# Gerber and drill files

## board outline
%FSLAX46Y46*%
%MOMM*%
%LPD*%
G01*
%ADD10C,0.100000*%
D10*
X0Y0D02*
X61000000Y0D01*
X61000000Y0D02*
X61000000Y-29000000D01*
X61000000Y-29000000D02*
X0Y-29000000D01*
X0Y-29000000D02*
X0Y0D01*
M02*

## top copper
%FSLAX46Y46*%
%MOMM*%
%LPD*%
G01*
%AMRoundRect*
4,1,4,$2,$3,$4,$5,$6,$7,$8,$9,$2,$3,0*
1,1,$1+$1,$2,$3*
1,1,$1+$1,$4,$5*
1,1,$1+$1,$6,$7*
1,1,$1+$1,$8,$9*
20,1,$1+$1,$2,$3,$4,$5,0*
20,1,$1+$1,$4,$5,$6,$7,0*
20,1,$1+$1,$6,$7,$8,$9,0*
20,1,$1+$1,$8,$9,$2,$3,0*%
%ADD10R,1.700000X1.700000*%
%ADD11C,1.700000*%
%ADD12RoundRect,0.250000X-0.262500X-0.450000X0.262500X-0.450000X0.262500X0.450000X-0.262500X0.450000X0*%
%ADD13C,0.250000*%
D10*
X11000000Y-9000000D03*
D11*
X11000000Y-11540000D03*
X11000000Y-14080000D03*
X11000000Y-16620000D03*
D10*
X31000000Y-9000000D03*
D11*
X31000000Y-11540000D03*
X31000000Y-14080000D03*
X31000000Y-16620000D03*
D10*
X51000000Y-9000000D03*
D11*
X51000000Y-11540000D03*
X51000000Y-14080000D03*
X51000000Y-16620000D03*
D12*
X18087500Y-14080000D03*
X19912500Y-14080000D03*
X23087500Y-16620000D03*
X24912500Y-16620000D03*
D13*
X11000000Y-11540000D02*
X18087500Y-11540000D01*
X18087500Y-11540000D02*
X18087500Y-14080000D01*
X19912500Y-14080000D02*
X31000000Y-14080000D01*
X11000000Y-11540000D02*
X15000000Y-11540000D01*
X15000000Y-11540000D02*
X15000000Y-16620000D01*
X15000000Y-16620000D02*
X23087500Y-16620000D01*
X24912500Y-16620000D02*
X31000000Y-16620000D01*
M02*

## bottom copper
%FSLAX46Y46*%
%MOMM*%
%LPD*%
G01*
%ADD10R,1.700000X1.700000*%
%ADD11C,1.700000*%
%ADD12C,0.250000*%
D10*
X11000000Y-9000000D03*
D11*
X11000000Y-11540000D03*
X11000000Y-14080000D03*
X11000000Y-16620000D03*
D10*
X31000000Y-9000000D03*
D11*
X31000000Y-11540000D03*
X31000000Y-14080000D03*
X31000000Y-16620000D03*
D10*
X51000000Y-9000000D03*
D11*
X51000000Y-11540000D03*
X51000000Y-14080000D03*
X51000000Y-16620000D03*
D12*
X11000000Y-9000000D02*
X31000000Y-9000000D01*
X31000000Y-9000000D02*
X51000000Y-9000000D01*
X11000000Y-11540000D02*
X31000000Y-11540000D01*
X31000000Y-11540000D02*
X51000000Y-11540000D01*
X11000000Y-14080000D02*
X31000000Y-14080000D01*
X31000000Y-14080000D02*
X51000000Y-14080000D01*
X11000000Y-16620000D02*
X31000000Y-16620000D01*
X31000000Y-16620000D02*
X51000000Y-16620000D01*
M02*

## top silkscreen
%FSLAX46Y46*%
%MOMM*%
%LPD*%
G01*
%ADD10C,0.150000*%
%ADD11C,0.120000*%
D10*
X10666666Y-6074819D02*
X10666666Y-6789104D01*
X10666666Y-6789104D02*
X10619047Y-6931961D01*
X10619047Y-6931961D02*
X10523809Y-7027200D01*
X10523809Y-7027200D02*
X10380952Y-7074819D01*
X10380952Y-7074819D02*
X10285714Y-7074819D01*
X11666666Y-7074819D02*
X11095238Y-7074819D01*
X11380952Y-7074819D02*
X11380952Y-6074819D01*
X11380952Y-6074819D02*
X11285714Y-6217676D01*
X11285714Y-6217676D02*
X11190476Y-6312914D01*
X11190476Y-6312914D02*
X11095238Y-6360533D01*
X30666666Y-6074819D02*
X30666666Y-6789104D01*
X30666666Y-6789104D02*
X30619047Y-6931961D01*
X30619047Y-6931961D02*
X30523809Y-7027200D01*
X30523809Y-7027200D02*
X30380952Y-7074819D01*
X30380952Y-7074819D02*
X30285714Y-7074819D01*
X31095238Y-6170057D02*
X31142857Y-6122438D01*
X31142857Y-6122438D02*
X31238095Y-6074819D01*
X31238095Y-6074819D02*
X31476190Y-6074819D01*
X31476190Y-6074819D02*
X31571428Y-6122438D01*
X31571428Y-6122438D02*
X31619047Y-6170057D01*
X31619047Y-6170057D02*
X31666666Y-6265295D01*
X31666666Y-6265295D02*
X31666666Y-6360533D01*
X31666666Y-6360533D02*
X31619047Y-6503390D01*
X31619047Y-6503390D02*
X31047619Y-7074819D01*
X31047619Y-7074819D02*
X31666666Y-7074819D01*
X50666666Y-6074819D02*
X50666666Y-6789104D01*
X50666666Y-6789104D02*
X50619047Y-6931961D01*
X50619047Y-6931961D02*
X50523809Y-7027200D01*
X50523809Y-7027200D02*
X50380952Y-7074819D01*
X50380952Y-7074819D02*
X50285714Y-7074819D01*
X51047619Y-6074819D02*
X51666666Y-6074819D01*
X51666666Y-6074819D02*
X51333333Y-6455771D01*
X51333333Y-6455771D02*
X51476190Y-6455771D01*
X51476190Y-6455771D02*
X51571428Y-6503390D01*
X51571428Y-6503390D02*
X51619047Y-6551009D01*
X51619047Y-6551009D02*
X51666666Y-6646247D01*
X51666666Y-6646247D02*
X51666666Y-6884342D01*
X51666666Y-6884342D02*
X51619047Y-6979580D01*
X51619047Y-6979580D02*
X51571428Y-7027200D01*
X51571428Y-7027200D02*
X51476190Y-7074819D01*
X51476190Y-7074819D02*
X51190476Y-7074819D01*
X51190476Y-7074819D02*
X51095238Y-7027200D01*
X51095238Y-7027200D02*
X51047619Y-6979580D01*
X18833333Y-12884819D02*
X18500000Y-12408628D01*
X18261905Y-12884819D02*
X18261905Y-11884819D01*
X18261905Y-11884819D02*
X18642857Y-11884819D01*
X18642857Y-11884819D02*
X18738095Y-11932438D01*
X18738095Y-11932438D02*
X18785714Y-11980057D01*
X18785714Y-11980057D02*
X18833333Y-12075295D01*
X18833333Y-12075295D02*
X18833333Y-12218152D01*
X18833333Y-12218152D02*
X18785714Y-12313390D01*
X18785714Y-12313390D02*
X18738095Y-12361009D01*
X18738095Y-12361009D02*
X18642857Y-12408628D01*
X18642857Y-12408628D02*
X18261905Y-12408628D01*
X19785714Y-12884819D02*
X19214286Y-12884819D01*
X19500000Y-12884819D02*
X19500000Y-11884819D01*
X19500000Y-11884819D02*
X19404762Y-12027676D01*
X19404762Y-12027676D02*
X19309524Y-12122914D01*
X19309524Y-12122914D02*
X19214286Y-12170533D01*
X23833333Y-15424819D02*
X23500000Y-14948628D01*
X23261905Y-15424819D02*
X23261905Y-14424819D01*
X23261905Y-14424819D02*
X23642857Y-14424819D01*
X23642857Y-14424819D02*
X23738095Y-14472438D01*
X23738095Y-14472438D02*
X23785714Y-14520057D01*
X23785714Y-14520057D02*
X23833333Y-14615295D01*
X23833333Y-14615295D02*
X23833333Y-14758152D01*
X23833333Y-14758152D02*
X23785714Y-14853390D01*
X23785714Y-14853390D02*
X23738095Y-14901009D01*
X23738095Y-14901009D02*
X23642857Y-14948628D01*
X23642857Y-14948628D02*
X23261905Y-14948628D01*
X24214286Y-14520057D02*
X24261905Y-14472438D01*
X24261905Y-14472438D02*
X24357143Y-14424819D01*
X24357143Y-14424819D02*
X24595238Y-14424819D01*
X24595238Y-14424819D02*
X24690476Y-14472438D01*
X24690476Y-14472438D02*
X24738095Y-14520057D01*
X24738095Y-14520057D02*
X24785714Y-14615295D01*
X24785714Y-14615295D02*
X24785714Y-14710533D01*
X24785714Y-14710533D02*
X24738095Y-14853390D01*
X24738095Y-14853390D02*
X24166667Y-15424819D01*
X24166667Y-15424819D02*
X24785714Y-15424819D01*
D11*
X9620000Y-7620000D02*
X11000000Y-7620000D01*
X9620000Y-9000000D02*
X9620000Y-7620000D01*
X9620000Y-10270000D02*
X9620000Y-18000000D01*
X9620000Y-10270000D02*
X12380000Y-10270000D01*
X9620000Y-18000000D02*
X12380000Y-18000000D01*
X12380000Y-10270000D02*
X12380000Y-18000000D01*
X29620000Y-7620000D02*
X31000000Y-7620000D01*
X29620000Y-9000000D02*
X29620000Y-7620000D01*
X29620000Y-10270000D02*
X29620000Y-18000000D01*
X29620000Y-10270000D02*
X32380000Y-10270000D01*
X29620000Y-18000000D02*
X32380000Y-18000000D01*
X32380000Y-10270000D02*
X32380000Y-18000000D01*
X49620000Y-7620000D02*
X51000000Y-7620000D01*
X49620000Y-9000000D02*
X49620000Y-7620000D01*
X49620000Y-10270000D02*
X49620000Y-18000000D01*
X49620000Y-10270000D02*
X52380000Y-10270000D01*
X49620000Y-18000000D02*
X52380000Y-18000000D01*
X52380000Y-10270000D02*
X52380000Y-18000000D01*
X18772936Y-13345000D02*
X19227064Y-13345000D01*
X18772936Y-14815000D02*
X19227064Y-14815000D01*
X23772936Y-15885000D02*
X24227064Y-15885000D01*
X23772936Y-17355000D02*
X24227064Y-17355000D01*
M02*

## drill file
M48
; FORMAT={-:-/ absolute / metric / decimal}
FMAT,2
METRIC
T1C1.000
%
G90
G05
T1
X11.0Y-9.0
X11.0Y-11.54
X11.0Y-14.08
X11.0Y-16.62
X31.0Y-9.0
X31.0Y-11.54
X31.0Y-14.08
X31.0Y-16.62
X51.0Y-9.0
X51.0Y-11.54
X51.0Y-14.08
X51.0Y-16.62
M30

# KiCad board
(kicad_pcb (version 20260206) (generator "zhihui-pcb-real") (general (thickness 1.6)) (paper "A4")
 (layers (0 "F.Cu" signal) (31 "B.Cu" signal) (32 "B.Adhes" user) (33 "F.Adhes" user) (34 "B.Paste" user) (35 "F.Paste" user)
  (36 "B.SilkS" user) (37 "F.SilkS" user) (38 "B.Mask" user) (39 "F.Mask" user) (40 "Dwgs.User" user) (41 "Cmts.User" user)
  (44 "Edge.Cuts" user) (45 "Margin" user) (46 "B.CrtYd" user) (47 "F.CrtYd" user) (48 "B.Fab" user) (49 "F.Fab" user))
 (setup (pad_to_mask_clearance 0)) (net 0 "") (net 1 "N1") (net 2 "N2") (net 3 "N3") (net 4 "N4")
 (gr_line (start 0 0) (end 61 0) (stroke (width 0.1) (type default)) (layer "Edge.Cuts"))
 (gr_line (start 61 0) (end 61 29) (stroke (width 0.1) (type default)) (layer "Edge.Cuts"))
 (gr_line (start 61 29) (end 0 29) (stroke (width 0.1) (type default)) (layer "Edge.Cuts"))
 (gr_line (start 0 29) (end 0 0) (stroke (width 0.1) (type default)) (layer "Edge.Cuts"))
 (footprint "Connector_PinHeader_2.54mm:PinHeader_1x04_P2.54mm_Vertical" (layer "F.Cu")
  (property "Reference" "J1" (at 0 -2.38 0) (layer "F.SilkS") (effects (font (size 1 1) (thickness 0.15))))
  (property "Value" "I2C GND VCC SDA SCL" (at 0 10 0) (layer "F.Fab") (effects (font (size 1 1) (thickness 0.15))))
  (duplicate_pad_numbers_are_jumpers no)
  (fp_line (start -1.38 -1.38) (end 0 -1.38) (stroke (width 0.12) (type solid)) (layer "F.SilkS"))
  (fp_line (start -1.38 0) (end -1.38 -1.38) (stroke (width 0.12) (type solid)) (layer "F.SilkS"))
  (fp_line (start -1.38 1.27) (end -1.38 9) (stroke (width 0.12) (type solid)) (layer "F.SilkS"))
  (fp_line (start -1.38 1.27) (end 1.38 1.27) (stroke (width 0.12) (type solid)) (layer "F.SilkS"))
  (fp_line (start -1.38 9) (end 1.38 9) (stroke (width 0.12) (type solid)) (layer "F.SilkS"))
  (fp_line (start 1.38 1.27) (end 1.38 9) (stroke (width 0.12) (type solid)) (layer "F.SilkS"))
  (pad "1" thru_hole rect (at 0 0) (size 1.7 1.7) (drill 1) (layers "*.Cu" "*.Mask") (remove_unused_layers no) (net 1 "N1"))
  (pad "2" thru_hole circle (at 0 2.54) (size 1.7 1.7) (drill 1) (layers "*.Cu" "*.Mask") (remove_unused_layers no) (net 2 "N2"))
  (pad "3" thru_hole circle (at 0 5.08) (size 1.7 1.7) (drill 1) (layers "*.Cu" "*.Mask") (remove_unused_layers no) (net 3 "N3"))
  (pad "4" thru_hole circle (at 0 7.62) (size 1.7 1.7) (drill 1) (layers "*.Cu" "*.Mask") (remove_unused_layers no) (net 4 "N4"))
  (at 11 9 0))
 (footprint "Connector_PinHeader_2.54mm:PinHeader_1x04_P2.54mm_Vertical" (layer "F.Cu")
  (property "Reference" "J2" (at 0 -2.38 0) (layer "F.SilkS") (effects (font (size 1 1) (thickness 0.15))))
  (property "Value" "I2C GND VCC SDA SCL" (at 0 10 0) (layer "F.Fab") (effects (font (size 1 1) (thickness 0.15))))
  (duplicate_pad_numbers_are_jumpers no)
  (fp_line (start -1.38 -1.38) (end 0 -1.38) (stroke (width 0.12) (type solid)) (layer "F.SilkS"))
  (fp_line (start -1.38 0) (end -1.38 -1.38) (stroke (width 0.12) (type solid)) (layer "F.SilkS"))
  (fp_line (start -1.38 1.27) (end -1.38 9) (stroke (width 0.12) (type solid)) (layer "F.SilkS"))
  (fp_line (start -1.38 1.27) (end 1.38 1.27) (stroke (width 0.12) (type solid)) (layer "F.SilkS"))
  (fp_line (start -1.38 9) (end 1.38 9) (stroke (width 0.12) (type solid)) (layer "F.SilkS"))
  (fp_line (start 1.38 1.27) (end 1.38 9) (stroke (width 0.12) (type solid)) (layer "F.SilkS"))
  (pad "1" thru_hole rect (at 0 0) (size 1.7 1.7) (drill 1) (layers "*.Cu" "*.Mask") (remove_unused_layers no) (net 1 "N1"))
  (pad "2" thru_hole circle (at 0 2.54) (size 1.7 1.7) (drill 1) (layers "*.Cu" "*.Mask") (remove_unused_layers no) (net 2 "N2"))
  (pad "3" thru_hole circle (at 0 5.08) (size 1.7 1.7) (drill 1) (layers "*.Cu" "*.Mask") (remove_unused_layers no) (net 3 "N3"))
  (pad "4" thru_hole circle (at 0 7.62) (size 1.7 1.7) (drill 1) (layers "*.Cu" "*.Mask") (remove_unused_layers no) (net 4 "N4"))
  (at 31 9 0))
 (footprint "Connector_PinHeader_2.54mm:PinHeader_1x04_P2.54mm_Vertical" (layer "F.Cu")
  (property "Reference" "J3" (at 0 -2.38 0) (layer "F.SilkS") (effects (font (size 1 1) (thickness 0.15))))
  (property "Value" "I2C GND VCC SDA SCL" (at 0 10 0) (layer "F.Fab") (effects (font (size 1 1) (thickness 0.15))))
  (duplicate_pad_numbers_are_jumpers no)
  (fp_line (start -1.38 -1.38) (end 0 -1.38) (stroke (width 0.12) (type solid)) (layer "F.SilkS"))
  (fp_line (start -1.38 0) (end -1.38 -1.38) (stroke (width 0.12) (type solid)) (layer "F.SilkS"))
  (fp_line (start -1.38 1.27) (end -1.38 9) (stroke (width 0.12) (type solid)) (layer "F.SilkS"))
  (fp_line (start -1.38 1.27) (end 1.38 1.27) (stroke (width 0.12) (type solid)) (layer "F.SilkS"))
  (fp_line (start -1.38 9) (end 1.38 9) (stroke (width 0.12) (type solid)) (layer "F.SilkS"))
  (fp_line (start 1.38 1.27) (end 1.38 9) (stroke (width 0.12) (type solid)) (layer "F.SilkS"))
  (pad "1" thru_hole rect (at 0 0) (size 1.7 1.7) (drill 1) (layers "*.Cu" "*.Mask") (remove_unused_layers no) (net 1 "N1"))
  (pad "2" thru_hole circle (at 0 2.54) (size 1.7 1.7) (drill 1) (layers "*.Cu" "*.Mask") (remove_unused_layers no) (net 2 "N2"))
  (pad "3" thru_hole circle (at 0 5.08) (size 1.7 1.7) (drill 1) (layers "*.Cu" "*.Mask") (remove_unused_layers no) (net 3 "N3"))
  (pad "4" thru_hole circle (at 0 7.62) (size 1.7 1.7) (drill 1) (layers "*.Cu" "*.Mask") (remove_unused_layers no) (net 4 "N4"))
  (at 51 9 0))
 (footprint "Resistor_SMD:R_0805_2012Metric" (layer "F.Cu")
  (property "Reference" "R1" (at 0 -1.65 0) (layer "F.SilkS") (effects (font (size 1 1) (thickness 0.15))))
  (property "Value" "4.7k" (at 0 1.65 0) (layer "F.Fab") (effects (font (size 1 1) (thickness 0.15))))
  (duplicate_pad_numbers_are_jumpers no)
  (fp_line (start -0.227064 -0.735) (end 0.227064 -0.735) (stroke (width 0.12) (type solid)) (layer "F.SilkS"))
  (fp_line (start -0.227064 0.735) (end 0.227064 0.735) (stroke (width 0.12) (type solid)) (layer "F.SilkS"))
  (pad "1" smd roundrect (at -0.9125 0) (size 1.025 1.4) (layers "F.Cu" "F.Mask" "F.Paste") (roundrect_rratio 0.243902) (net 2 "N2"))
  (pad "2" smd roundrect (at 0.9125 0) (size 1.025 1.4) (layers "F.Cu" "F.Mask" "F.Paste") (roundrect_rratio 0.243902) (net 3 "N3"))
  (at 19 14.08 0))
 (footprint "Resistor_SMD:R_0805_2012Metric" (layer "F.Cu")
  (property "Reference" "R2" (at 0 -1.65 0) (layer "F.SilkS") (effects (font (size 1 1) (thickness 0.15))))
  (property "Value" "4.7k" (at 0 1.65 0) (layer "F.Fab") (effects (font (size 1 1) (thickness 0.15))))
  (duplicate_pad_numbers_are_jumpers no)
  (fp_line (start -0.227064 -0.735) (end 0.227064 -0.735) (stroke (width 0.12) (type solid)) (layer "F.SilkS"))
  (fp_line (start -0.227064 0.735) (end 0.227064 0.735) (stroke (width 0.12) (type solid)) (layer "F.SilkS"))
  (pad "1" smd roundrect (at -0.9125 0) (size 1.025 1.4) (layers "F.Cu" "F.Mask" "F.Paste") (roundrect_rratio 0.243902) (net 2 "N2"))
  (pad "2" smd roundrect (at 0.9125 0) (size 1.025 1.4) (layers "F.Cu" "F.Mask" "F.Paste") (roundrect_rratio 0.243902) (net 4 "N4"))
  (at 24 16.62 0))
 (segment (start 11 9) (end 31 9) (width 0.25) (layer "B.Cu") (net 1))
 (segment (start 31 9) (end 51 9) (width 0.25) (layer "B.Cu") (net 1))
 (segment (start 11 11.54) (end 31 11.54) (width 0.25) (layer "B.Cu") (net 2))
 (segment (start 31 11.54) (end 51 11.54) (width 0.25) (layer "B.Cu") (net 2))
 (segment (start 11 14.08) (end 31 14.08) (width 0.25) (layer "B.Cu") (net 3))
 (segment (start 31 14.08) (end 51 14.08) (width 0.25) (layer "B.Cu") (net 3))
 (segment (start 11 16.62) (end 31 16.62) (width 0.25) (layer "B.Cu") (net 4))
 (segment (start 31 16.62) (end 51 16.62) (width 0.25) (layer "B.Cu") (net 4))
 (segment (start 11 11.54) (end 18.0875 11.54) (width 0.25) (layer "F.Cu") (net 2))
 (segment (start 18.0875 11.54) (end 18.0875 14.08) (width 0.25) (layer "F.Cu") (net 2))
 (segment (start 19.9125 14.08) (end 31 14.08) (width 0.25) (layer "F.Cu") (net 3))
 (segment (start 11 11.54) (end 15 11.54) (width 0.25) (layer "F.Cu") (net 2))
 (segment (start 15 11.54) (end 15 16.62) (width 0.25) (layer "F.Cu") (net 2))
 (segment (start 15 16.62) (end 23.0875 16.62) (width 0.25) (layer "F.Cu") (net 2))
 (segment (start 24.9125 16.62) (end 31 16.62) (width 0.25) (layer "F.Cu") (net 4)))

